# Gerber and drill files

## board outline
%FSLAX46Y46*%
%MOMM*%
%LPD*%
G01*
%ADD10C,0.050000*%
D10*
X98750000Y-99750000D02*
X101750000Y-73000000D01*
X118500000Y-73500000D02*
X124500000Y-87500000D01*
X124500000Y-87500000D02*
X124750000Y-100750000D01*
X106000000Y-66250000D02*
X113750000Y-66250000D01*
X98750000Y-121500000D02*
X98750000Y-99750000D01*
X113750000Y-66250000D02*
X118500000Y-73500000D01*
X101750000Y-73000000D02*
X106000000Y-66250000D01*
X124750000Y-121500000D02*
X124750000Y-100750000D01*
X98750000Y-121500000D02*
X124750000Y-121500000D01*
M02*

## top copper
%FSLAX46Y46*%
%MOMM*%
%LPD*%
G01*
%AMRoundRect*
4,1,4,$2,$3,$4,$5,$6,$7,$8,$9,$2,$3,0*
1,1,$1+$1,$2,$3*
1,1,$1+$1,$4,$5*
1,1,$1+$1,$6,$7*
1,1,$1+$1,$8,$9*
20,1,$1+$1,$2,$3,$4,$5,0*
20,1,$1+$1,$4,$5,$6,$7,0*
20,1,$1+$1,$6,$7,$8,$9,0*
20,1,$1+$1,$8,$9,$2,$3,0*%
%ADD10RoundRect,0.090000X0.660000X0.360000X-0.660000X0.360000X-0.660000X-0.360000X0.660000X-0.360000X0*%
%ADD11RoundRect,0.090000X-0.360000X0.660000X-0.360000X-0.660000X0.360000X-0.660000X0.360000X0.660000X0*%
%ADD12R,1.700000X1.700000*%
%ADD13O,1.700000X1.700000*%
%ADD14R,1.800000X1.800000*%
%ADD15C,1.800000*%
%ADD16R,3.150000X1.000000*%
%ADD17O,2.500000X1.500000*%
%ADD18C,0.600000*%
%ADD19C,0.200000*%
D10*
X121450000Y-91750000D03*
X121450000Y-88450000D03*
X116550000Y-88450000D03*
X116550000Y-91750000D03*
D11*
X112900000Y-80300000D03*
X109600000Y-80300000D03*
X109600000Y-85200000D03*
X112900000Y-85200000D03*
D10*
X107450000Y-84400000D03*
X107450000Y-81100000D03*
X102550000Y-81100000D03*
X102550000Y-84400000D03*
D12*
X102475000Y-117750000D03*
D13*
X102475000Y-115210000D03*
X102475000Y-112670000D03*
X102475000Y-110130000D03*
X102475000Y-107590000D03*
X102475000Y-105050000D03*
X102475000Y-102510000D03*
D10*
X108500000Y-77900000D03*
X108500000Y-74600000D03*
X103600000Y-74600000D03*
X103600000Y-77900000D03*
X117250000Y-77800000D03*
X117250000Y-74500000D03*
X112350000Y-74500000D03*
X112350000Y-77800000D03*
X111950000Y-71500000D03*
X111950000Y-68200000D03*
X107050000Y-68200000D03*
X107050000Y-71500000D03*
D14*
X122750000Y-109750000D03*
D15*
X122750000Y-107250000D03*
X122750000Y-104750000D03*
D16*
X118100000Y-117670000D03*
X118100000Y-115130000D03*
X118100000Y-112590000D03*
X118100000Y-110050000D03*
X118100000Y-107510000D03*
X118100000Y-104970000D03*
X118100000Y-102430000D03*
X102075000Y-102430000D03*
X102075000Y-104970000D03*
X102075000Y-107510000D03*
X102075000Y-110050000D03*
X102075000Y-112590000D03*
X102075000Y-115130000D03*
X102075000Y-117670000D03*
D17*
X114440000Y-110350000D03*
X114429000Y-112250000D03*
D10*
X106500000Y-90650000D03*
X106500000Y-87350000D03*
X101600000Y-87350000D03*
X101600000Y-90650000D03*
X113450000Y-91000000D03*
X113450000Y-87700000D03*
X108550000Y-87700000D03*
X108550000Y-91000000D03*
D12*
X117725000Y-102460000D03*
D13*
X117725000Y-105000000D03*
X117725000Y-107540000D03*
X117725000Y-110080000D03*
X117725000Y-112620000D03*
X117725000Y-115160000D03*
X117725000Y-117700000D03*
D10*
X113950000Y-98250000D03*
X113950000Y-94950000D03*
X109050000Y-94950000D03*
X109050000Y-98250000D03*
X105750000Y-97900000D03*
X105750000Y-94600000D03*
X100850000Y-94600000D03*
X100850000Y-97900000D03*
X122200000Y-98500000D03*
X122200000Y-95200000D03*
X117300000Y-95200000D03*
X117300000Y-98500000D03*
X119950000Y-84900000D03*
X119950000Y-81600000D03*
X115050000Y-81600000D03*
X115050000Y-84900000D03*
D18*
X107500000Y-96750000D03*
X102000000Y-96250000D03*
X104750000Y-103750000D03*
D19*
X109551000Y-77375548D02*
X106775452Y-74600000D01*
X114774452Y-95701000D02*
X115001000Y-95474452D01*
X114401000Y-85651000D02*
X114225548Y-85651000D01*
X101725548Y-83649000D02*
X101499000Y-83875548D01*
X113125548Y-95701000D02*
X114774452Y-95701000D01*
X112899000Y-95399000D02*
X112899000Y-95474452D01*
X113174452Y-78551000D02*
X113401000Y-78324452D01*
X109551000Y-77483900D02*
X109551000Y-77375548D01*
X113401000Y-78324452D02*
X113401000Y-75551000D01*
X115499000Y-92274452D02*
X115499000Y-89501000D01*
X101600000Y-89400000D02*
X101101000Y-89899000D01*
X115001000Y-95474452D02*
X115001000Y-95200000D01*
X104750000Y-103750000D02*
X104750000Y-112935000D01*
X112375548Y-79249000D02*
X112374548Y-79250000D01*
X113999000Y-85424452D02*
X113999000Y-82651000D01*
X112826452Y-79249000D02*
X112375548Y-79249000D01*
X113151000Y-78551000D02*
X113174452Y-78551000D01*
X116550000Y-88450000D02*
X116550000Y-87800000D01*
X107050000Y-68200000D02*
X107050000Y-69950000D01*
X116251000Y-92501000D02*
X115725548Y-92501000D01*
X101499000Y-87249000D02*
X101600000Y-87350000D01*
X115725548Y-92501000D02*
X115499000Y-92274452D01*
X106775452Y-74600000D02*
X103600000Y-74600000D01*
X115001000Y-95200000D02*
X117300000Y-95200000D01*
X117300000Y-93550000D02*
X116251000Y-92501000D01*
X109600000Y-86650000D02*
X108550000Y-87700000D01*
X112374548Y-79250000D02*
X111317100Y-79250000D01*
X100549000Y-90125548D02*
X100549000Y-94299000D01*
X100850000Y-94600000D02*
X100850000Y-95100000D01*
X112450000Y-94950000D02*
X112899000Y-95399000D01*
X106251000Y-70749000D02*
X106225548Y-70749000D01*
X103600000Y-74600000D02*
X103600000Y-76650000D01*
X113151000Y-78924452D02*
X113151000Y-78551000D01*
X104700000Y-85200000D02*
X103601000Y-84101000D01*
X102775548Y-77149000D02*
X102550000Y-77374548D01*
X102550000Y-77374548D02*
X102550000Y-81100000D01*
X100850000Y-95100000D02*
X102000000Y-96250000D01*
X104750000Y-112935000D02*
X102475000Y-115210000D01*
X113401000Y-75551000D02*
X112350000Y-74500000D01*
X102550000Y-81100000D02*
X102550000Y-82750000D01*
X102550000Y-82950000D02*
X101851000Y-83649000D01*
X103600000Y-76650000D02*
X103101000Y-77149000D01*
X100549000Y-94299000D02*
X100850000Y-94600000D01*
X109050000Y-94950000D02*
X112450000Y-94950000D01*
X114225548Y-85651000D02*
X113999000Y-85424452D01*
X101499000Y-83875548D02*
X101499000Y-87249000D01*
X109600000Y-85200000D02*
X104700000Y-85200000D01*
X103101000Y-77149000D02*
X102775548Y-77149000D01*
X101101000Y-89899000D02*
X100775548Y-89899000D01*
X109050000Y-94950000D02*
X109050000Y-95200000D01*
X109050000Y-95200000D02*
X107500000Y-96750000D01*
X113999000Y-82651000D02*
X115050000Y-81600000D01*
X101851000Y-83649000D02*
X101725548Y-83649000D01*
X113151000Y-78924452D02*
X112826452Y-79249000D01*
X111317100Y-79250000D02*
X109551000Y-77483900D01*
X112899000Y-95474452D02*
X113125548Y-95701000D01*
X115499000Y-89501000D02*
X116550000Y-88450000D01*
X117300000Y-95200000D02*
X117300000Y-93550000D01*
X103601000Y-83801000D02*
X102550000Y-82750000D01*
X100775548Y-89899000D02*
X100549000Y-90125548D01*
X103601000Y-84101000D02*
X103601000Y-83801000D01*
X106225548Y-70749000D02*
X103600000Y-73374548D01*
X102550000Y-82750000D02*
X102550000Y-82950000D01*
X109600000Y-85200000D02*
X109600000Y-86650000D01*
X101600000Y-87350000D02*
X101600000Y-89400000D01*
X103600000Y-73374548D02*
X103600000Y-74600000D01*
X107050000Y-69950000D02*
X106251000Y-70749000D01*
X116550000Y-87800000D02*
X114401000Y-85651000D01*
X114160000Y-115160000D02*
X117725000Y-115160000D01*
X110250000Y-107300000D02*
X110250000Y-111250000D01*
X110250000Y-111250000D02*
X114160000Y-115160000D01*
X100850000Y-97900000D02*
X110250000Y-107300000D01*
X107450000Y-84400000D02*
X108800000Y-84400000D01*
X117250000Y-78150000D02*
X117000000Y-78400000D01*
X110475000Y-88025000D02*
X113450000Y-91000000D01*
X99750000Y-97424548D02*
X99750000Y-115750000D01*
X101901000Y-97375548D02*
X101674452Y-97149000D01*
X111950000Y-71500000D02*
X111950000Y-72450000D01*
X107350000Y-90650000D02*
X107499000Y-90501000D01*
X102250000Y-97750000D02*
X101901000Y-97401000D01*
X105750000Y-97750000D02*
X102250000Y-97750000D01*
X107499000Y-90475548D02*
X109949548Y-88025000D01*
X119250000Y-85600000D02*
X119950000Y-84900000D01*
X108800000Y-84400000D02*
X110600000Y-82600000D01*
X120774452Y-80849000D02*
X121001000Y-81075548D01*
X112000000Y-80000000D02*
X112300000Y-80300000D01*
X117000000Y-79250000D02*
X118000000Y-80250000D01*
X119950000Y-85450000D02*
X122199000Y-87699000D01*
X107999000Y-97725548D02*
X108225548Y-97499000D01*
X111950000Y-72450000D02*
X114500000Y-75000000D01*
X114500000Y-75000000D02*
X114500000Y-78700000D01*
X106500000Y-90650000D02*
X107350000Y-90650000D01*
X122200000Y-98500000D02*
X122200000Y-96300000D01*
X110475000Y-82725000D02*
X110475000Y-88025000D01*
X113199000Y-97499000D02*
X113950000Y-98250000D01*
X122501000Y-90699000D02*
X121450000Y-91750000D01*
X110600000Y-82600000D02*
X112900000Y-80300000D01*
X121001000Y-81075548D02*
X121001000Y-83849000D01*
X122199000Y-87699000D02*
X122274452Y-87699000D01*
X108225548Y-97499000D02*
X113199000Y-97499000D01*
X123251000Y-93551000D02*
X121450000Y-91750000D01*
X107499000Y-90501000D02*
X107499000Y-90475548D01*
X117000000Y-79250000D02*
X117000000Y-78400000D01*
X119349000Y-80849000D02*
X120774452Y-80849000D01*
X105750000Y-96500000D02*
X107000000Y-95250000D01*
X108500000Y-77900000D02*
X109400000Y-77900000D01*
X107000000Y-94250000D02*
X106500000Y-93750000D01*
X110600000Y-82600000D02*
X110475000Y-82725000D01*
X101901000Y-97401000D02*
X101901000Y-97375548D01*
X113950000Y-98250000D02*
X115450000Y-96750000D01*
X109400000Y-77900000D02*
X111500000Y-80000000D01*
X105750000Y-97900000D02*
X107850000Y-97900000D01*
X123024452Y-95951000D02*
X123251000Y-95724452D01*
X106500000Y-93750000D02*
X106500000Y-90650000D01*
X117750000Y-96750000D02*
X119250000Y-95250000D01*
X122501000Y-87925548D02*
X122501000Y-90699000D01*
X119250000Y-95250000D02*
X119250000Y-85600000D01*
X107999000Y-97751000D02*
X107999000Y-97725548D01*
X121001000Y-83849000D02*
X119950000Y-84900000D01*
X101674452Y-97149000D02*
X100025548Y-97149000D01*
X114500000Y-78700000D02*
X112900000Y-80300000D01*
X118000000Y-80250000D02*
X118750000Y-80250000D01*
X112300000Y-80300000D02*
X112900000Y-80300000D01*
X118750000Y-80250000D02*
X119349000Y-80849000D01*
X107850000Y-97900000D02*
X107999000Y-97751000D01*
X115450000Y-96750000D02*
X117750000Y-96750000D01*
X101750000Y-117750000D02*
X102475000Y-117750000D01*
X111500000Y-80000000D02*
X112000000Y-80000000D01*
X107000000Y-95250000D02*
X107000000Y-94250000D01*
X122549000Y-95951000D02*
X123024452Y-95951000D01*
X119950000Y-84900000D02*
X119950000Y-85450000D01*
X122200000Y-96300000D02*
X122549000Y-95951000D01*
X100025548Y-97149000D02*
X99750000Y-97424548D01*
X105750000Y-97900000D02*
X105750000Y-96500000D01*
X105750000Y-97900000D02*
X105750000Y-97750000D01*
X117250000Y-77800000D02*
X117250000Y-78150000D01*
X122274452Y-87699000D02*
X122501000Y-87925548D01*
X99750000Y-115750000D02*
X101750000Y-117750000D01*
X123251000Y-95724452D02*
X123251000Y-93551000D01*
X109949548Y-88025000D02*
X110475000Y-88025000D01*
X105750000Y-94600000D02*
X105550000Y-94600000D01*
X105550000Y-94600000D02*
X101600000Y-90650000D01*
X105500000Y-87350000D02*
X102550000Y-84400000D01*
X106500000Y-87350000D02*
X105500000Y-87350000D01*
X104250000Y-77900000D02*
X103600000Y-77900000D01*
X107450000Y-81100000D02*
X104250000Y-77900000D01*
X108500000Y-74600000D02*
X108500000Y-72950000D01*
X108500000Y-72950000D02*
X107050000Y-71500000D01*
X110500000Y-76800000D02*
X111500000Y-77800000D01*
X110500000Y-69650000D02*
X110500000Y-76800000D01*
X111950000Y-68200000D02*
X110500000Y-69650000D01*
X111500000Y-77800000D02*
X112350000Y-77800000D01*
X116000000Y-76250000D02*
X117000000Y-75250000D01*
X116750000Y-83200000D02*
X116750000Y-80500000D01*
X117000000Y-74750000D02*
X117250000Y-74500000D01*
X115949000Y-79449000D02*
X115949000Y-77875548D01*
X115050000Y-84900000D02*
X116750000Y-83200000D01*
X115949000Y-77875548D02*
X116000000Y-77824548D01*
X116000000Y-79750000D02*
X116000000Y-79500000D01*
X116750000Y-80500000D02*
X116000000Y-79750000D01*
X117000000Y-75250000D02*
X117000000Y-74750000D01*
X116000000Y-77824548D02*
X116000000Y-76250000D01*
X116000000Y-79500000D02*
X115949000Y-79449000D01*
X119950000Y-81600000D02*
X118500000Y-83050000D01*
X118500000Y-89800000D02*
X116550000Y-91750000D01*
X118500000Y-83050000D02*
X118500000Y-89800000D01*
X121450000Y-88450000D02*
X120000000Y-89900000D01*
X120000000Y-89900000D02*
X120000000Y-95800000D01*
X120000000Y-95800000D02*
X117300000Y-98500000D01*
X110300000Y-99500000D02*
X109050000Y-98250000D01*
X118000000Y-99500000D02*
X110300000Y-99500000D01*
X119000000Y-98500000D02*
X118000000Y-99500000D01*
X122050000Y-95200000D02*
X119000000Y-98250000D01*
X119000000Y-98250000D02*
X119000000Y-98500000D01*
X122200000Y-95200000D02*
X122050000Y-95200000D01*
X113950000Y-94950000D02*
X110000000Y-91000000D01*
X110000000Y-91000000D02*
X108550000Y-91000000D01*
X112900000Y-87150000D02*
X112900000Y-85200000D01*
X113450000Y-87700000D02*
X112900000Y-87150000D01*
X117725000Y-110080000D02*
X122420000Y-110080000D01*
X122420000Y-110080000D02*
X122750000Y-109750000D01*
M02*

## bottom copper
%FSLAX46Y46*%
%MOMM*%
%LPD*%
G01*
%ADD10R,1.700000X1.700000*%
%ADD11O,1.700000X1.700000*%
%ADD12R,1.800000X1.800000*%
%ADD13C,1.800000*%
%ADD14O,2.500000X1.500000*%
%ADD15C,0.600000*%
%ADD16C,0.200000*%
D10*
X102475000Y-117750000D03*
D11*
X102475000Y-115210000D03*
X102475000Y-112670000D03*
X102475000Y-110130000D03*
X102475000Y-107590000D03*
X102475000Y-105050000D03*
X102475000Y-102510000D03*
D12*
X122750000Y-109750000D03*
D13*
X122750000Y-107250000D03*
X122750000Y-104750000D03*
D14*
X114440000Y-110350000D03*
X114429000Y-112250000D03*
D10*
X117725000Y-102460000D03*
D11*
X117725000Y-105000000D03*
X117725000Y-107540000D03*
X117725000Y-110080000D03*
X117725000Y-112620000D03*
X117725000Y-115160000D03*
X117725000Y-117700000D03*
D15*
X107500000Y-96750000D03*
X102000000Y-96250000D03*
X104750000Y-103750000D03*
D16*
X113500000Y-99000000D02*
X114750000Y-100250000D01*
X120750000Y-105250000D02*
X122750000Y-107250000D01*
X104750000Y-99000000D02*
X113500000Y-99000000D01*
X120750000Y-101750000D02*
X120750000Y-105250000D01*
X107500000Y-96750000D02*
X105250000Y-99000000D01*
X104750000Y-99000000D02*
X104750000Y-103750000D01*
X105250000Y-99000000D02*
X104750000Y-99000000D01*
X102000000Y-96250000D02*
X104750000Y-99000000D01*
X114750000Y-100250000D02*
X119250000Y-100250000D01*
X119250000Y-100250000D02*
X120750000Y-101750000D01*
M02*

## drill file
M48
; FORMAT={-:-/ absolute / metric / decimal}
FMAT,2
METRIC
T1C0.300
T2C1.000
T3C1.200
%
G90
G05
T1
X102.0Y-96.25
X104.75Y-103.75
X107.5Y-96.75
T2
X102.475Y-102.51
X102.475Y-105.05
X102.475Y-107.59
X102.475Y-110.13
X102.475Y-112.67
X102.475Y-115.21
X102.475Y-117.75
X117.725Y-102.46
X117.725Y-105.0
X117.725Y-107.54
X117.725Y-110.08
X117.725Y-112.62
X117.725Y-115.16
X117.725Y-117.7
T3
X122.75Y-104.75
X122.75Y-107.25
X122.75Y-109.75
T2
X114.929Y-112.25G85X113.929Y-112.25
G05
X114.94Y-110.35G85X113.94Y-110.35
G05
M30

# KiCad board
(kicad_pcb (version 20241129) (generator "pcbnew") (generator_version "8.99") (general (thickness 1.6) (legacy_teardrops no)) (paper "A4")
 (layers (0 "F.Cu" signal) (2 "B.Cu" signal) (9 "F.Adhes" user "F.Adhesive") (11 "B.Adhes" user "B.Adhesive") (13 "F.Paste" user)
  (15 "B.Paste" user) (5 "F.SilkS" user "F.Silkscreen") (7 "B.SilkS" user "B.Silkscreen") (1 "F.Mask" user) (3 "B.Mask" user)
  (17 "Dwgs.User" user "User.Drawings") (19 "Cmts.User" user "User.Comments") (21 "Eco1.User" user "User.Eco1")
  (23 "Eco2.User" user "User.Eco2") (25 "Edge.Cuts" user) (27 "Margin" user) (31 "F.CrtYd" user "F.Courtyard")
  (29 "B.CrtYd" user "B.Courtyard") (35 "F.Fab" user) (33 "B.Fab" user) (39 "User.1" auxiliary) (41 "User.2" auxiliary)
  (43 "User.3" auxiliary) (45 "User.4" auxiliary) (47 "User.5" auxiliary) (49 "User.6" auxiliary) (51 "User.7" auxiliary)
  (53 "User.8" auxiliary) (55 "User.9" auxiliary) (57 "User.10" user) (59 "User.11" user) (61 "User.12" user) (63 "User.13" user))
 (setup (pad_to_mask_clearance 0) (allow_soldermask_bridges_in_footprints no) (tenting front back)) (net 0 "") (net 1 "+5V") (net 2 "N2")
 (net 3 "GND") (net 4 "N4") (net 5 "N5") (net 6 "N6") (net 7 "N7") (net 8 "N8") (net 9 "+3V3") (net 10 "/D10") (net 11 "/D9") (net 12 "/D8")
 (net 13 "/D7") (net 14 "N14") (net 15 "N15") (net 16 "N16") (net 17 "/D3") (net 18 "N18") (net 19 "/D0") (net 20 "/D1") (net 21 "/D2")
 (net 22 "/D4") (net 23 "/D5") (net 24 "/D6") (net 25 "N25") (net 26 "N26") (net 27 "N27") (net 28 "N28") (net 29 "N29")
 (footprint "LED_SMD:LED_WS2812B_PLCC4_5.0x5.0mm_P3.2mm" (layer "F.Cu") (at 119 90.1 180)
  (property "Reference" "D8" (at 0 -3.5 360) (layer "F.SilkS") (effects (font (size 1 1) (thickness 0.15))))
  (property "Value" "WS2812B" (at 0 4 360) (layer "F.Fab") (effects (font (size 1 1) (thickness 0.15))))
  (pad "1" smd roundrect (at -2.45 -1.65 180) (size 1.5 0.9) (layers "F.Cu" "F.Mask" "F.Paste") (roundrect_rratio 0.1) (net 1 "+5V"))
  (pad "2" smd roundrect (at -2.45 1.65 180) (size 1.5 0.9) (layers "F.Cu" "F.Mask" "F.Paste") (roundrect_rratio 0.1) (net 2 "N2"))
  (pad "3" smd roundrect (at 2.45 1.65 180) (size 1.5 0.9) (layers "F.Cu" "F.Mask" "F.Paste") (roundrect_rratio 0.1) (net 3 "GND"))
  (pad "4" smd roundrect (at 2.45 -1.65 180) (size 1.5 0.9) (layers "F.Cu" "F.Mask" "F.Paste") (roundrect_rratio 0.1) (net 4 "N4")))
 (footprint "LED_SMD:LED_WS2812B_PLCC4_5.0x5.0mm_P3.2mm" (layer "F.Cu") (at 111.25 82.75 -90)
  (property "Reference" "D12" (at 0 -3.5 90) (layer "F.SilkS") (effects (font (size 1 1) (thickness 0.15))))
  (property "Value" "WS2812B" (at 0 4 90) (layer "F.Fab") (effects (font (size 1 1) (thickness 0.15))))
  (pad "1" smd roundrect (at -2.45 -1.65 270) (size 1.5 0.9) (layers "F.Cu" "F.Mask" "F.Paste") (roundrect_rratio 0.1) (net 1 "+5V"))
  (pad "2" smd roundrect (at -2.45 1.65 270) (size 1.5 0.9) (layers "F.Cu" "F.Mask" "F.Paste") (roundrect_rratio 0.1) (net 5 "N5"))
  (pad "3" smd roundrect (at 2.45 1.65 270) (size 1.5 0.9) (layers "F.Cu" "F.Mask" "F.Paste") (roundrect_rratio 0.1) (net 3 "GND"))
  (pad "4" smd roundrect (at 2.45 -1.65 270) (size 1.5 0.9) (layers "F.Cu" "F.Mask" "F.Paste") (roundrect_rratio 0.1) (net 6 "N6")))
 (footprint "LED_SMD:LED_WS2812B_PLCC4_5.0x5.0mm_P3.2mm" (layer "F.Cu") (at 105 82.75 180)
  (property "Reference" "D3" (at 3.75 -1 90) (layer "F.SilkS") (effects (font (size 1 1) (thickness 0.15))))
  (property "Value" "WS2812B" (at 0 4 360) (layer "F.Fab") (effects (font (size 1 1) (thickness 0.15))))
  (pad "1" smd roundrect (at -2.45 -1.65 180) (size 1.5 0.9) (layers "F.Cu" "F.Mask" "F.Paste") (roundrect_rratio 0.1) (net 1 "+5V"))
  (pad "2" smd roundrect (at -2.45 1.65 180) (size 1.5 0.9) (layers "F.Cu" "F.Mask" "F.Paste") (roundrect_rratio 0.1) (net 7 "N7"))
  (pad "3" smd roundrect (at 2.45 1.65 180) (size 1.5 0.9) (layers "F.Cu" "F.Mask" "F.Paste") (roundrect_rratio 0.1) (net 3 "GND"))
  (pad "4" smd roundrect (at 2.45 -1.65 180) (size 1.5 0.9) (layers "F.Cu" "F.Mask" "F.Paste") (roundrect_rratio 0.1) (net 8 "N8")))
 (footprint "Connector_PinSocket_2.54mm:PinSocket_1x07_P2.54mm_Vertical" (layer "F.Cu") (at 102.475 117.75 180)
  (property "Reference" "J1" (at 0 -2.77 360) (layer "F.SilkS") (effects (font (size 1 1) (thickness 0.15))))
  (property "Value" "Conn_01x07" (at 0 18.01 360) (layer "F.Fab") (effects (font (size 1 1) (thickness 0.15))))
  (pad "1" thru_hole rect (at 0 0 180) (size 1.7 1.7) (drill 1) (layers "*.Cu" "*.Mask") (remove_unused_layers no) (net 1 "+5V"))
  (pad "2" thru_hole oval (at 0 2.54 180) (size 1.7 1.7) (drill 1) (layers "*.Cu" "*.Mask") (remove_unused_layers no) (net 3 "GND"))
  (pad "3" thru_hole oval (at 0 5.08 180) (size 1.7 1.7) (drill 1) (layers "*.Cu" "*.Mask") (remove_unused_layers no) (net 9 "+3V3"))
  (pad "4" thru_hole oval (at 0 7.62 180) (size 1.7 1.7) (drill 1) (layers "*.Cu" "*.Mask") (remove_unused_layers no) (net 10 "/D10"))
  (pad "5" thru_hole oval (at 0 10.16 180) (size 1.7 1.7) (drill 1) (layers "*.Cu" "*.Mask") (remove_unused_layers no) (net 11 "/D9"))
  (pad "6" thru_hole oval (at 0 12.7 180) (size 1.7 1.7) (drill 1) (layers "*.Cu" "*.Mask") (remove_unused_layers no) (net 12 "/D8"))
  (pad "7" thru_hole oval (at 0 15.24 180) (size 1.7 1.7) (drill 1) (layers "*.Cu" "*.Mask") (remove_unused_layers no) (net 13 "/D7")))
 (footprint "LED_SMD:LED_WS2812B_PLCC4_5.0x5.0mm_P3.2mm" (layer "F.Cu") (at 106.05 76.25 180)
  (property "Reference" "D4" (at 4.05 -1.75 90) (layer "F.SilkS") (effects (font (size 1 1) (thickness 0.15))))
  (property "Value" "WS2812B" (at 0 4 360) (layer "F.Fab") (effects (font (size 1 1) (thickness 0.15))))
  (pad "1" smd roundrect (at -2.45 -1.65 180) (size 1.5 0.9) (layers "F.Cu" "F.Mask" "F.Paste") (roundrect_rratio 0.1) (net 1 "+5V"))
  (pad "2" smd roundrect (at -2.45 1.65 180) (size 1.5 0.9) (layers "F.Cu" "F.Mask" "F.Paste") (roundrect_rratio 0.1) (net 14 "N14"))
  (pad "3" smd roundrect (at 2.45 1.65 180) (size 1.5 0.9) (layers "F.Cu" "F.Mask" "F.Paste") (roundrect_rratio 0.1) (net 3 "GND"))
  (pad "4" smd roundrect (at 2.45 -1.65 180) (size 1.5 0.9) (layers "F.Cu" "F.Mask" "F.Paste") (roundrect_rratio 0.1) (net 7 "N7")))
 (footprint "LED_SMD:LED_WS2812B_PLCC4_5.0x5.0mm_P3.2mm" (layer "F.Cu") (at 114.8 76.15 180)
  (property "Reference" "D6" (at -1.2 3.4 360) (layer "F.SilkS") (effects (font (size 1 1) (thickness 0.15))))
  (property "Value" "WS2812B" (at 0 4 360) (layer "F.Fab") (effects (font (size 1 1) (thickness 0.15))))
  (pad "1" smd roundrect (at -2.45 -1.65 180) (size 1.5 0.9) (layers "F.Cu" "F.Mask" "F.Paste") (roundrect_rratio 0.1) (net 1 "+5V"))
  (pad "2" smd roundrect (at -2.45 1.65 180) (size 1.5 0.9) (layers "F.Cu" "F.Mask" "F.Paste") (roundrect_rratio 0.1) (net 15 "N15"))
  (pad "3" smd roundrect (at 2.45 1.65 180) (size 1.5 0.9) (layers "F.Cu" "F.Mask" "F.Paste") (roundrect_rratio 0.1) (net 3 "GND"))
  (pad "4" smd roundrect (at 2.45 -1.65 180) (size 1.5 0.9) (layers "F.Cu" "F.Mask" "F.Paste") (roundrect_rratio 0.1) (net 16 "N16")))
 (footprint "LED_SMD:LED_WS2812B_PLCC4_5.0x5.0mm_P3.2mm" (layer "F.Cu") (at 109.5 69.85 180)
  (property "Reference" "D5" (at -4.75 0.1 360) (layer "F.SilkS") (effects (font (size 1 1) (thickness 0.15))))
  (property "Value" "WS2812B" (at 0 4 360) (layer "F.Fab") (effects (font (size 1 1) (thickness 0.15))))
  (pad "1" smd roundrect (at -2.45 -1.65 180) (size 1.5 0.9) (layers "F.Cu" "F.Mask" "F.Paste") (roundrect_rratio 0.1) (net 1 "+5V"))
  (pad "2" smd roundrect (at -2.45 1.65 180) (size 1.5 0.9) (layers "F.Cu" "F.Mask" "F.Paste") (roundrect_rratio 0.1) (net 16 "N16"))
  (pad "3" smd roundrect (at 2.45 1.65 180) (size 1.5 0.9) (layers "F.Cu" "F.Mask" "F.Paste") (roundrect_rratio 0.1) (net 3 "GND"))
  (pad "4" smd roundrect (at 2.45 -1.65 180) (size 1.5 0.9) (layers "F.Cu" "F.Mask" "F.Paste") (roundrect_rratio 0.1) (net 14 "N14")))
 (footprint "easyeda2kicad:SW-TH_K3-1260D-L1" (layer "F.Cu") (at 122.75 107.25 180)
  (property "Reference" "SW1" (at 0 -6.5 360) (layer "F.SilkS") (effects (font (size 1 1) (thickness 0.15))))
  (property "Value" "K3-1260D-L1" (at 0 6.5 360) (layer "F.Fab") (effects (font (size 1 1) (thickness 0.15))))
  (pad "1" thru_hole rect (at 0 -2.5 90) (size 1.8 1.8) (drill 1.199998) (layers "*.Cu" "*.Mask") (remove_unused_layers no) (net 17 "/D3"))
  (pad "2" thru_hole circle (at 0 0 90) (size 1.8 1.8) (drill 1.199998) (layers "*.Cu" "*.Mask") (remove_unused_layers no) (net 3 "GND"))
  (pad "3" thru_hole circle (at 0 2.5 90) (size 1.8 1.8) (drill 1.199998) (layers "*.Cu" "*.Mask") (remove_unused_layers no) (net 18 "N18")))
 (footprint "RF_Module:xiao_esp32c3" (layer "F.Cu") (at 109.5 108.25 180)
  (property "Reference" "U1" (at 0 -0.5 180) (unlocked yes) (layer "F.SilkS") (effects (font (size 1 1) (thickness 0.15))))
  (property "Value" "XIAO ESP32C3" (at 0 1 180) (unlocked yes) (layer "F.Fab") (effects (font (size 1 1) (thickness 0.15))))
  (pad "1" smd rect (at -8.6 -9.42 180) (size 3.15 1) (layers "F.Cu" "F.Mask" "F.Paste") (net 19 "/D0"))
  (pad "2" smd rect (at -8.6 -6.88 180) (size 3.15 1) (layers "F.Cu" "F.Mask" "F.Paste") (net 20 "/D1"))
  (pad "3" smd rect (at -8.6 -4.34 180) (size 3.15 1) (layers "F.Cu" "F.Mask" "F.Paste") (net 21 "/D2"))
  (pad "4" smd rect (at -8.6 -1.8 180) (size 3.15 1) (layers "F.Cu" "F.Mask" "F.Paste") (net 17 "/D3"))
  (pad "5" smd rect (at -8.6 0.74 180) (size 3.15 1) (layers "F.Cu" "F.Mask" "F.Paste") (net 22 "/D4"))
  (pad "6" smd rect (at -8.6 3.28 180) (size 3.15 1) (layers "F.Cu" "F.Mask" "F.Paste") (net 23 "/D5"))
  (pad "7" smd rect (at -8.6 5.82 180) (size 3.15 1) (layers "F.Cu" "F.Mask" "F.Paste") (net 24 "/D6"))
  (pad "8" smd rect (at 7.425 5.82 180) (size 3.15 1) (layers "F.Cu" "F.Mask" "F.Paste") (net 13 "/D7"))
  (pad "9" smd rect (at 7.425 3.28 180) (size 3.15 1) (layers "F.Cu" "F.Mask" "F.Paste") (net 12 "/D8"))
  (pad "10" smd rect (at 7.425 0.74 180) (size 3.15 1) (layers "F.Cu" "F.Mask" "F.Paste") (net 11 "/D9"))
  (pad "11" smd rect (at 7.425 -1.8 180) (size 3.15 1) (layers "F.Cu" "F.Mask" "F.Paste") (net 10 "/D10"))
  (pad "12" smd rect (at 7.425 -4.34 180) (size 3.15 1) (layers "F.Cu" "F.Mask" "F.Paste") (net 9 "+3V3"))
  (pad "13" smd rect (at 7.425 -6.88 180) (size 3.15 1) (layers "F.Cu" "F.Mask" "F.Paste") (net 3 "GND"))
  (pad "14" smd rect (at 7.425 -9.42 180) (size 3.15 1) (layers "F.Cu" "F.Mask" "F.Paste") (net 1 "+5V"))
  (pad "B+" thru_hole oval (at -4.94 -2.1 180) (size 2.5 1.5) (drill oval 2 1) (layers "*.Cu" "*.Mask") (remove_unused_layers no)
   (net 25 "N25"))
  (pad "B-" thru_hole oval (at -4.929 -4 180) (size 2.5 1.5) (drill oval 2 1) (layers "*.Cu" "*.Mask") (remove_unused_layers no)
   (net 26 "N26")))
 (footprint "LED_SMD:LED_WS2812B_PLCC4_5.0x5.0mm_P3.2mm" (layer "F.Cu") (at 104.05 89 180)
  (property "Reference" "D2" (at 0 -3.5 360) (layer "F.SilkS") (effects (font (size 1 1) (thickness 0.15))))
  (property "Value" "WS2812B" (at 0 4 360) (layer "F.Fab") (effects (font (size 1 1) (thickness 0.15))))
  (pad "1" smd roundrect (at -2.45 -1.65 180) (size 1.5 0.9) (layers "F.Cu" "F.Mask" "F.Paste") (roundrect_rratio 0.1) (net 1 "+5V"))
  (pad "2" smd roundrect (at -2.45 1.65 180) (size 1.5 0.9) (layers "F.Cu" "F.Mask" "F.Paste") (roundrect_rratio 0.1) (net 8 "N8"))
  (pad "3" smd roundrect (at 2.45 1.65 180) (size 1.5 0.9) (layers "F.Cu" "F.Mask" "F.Paste") (roundrect_rratio 0.1) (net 3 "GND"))
  (pad "4" smd roundrect (at 2.45 -1.65 180) (size 1.5 0.9) (layers "F.Cu" "F.Mask" "F.Paste") (roundrect_rratio 0.1) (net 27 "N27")))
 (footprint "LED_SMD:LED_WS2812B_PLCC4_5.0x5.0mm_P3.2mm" (layer "F.Cu") (at 111 89.35 180)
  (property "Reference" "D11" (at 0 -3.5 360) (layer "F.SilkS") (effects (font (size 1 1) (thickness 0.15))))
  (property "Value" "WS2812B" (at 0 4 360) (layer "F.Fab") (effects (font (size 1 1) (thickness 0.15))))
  (pad "1" smd roundrect (at -2.45 -1.65 180) (size 1.5 0.9) (layers "F.Cu" "F.Mask" "F.Paste") (roundrect_rratio 0.1) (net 1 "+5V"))
  (pad "2" smd roundrect (at -2.45 1.65 180) (size 1.5 0.9) (layers "F.Cu" "F.Mask" "F.Paste") (roundrect_rratio 0.1) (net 6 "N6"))
  (pad "3" smd roundrect (at 2.45 1.65 180) (size 1.5 0.9) (layers "F.Cu" "F.Mask" "F.Paste") (roundrect_rratio 0.1) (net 3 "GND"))
  (pad "4" smd roundrect (at 2.45 -1.65 180) (size 1.5 0.9) (layers "F.Cu" "F.Mask" "F.Paste") (roundrect_rratio 0.1) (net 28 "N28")))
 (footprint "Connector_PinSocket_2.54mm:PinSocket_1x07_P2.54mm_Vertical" (layer "F.Cu") (at 117.725 102.46)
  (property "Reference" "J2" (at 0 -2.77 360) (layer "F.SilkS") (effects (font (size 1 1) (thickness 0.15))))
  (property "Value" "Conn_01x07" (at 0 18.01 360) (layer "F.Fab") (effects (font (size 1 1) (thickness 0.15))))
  (pad "1" thru_hole rect (at 0 0) (size 1.7 1.7) (drill 1) (layers "*.Cu" "*.Mask") (remove_unused_layers no) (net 24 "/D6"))
  (pad "2" thru_hole oval (at 0 2.54) (size 1.7 1.7) (drill 1) (layers "*.Cu" "*.Mask") (remove_unused_layers no) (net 23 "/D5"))
  (pad "3" thru_hole oval (at 0 5.08) (size 1.7 1.7) (drill 1) (layers "*.Cu" "*.Mask") (remove_unused_layers no) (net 22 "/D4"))
  (pad "4" thru_hole oval (at 0 7.62) (size 1.7 1.7) (drill 1) (layers "*.Cu" "*.Mask") (remove_unused_layers no) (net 17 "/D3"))
  (pad "5" thru_hole oval (at 0 10.16) (size 1.7 1.7) (drill 1) (layers "*.Cu" "*.Mask") (remove_unused_layers no) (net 21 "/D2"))
  (pad "6" thru_hole oval (at 0 12.7) (size 1.7 1.7) (drill 1) (layers "*.Cu" "*.Mask") (remove_unused_layers no) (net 20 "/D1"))
  (pad "7" thru_hole oval (at 0 15.24) (size 1.7 1.7) (drill 1) (layers "*.Cu" "*.Mask") (remove_unused_layers no) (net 19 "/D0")))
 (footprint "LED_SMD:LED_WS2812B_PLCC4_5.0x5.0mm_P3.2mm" (layer "F.Cu") (at 111.5 96.6 180)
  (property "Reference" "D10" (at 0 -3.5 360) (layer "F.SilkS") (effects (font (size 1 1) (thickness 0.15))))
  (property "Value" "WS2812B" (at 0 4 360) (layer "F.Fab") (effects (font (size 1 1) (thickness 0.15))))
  (pad "1" smd roundrect (at -2.45 -1.65 180) (size 1.5 0.9) (layers "F.Cu" "F.Mask" "F.Paste") (roundrect_rratio 0.1) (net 1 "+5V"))
  (pad "2" smd roundrect (at -2.45 1.65 180) (size 1.5 0.9) (layers "F.Cu" "F.Mask" "F.Paste") (roundrect_rratio 0.1) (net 28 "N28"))
  (pad "3" smd roundrect (at 2.45 1.65 180) (size 1.5 0.9) (layers "F.Cu" "F.Mask" "F.Paste") (roundrect_rratio 0.1) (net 3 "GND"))
  (pad "4" smd roundrect (at 2.45 -1.65 180) (size 1.5 0.9) (layers "F.Cu" "F.Mask" "F.Paste") (roundrect_rratio 0.1) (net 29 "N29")))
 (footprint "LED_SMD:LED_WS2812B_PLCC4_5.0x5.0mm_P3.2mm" (layer "F.Cu") (at 103.3 96.25 180)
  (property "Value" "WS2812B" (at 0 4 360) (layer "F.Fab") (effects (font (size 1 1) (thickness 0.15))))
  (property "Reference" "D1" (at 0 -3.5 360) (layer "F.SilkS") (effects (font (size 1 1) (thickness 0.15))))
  (pad "1" smd roundrect (at -2.45 -1.65 180) (size 1.5 0.9) (layers "F.Cu" "F.Mask" "F.Paste") (roundrect_rratio 0.1) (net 1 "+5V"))
  (pad "2" smd roundrect (at -2.45 1.65 180) (size 1.5 0.9) (layers "F.Cu" "F.Mask" "F.Paste") (roundrect_rratio 0.1) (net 27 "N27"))
  (pad "3" smd roundrect (at 2.45 1.65 180) (size 1.5 0.9) (layers "F.Cu" "F.Mask" "F.Paste") (roundrect_rratio 0.1) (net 3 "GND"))
  (pad "4" smd roundrect (at 2.45 -1.65 180) (size 1.5 0.9) (layers "F.Cu" "F.Mask" "F.Paste") (roundrect_rratio 0.1) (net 20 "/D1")))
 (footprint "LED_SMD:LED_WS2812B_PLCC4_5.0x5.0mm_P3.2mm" (layer "F.Cu") (at 119.75 96.85 180)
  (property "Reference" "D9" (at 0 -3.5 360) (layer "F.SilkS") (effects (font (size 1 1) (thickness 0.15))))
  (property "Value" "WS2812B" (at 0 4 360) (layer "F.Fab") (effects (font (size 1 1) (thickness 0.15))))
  (pad "1" smd roundrect (at -2.45 -1.65 180) (size 1.5 0.9) (layers "F.Cu" "F.Mask" "F.Paste") (roundrect_rratio 0.1) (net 1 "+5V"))
  (pad "2" smd roundrect (at -2.45 1.65 180) (size 1.5 0.9) (layers "F.Cu" "F.Mask" "F.Paste") (roundrect_rratio 0.1) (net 29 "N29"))
  (pad "3" smd roundrect (at 2.45 1.65 180) (size 1.5 0.9) (layers "F.Cu" "F.Mask" "F.Paste") (roundrect_rratio 0.1) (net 3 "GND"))
  (pad "4" smd roundrect (at 2.45 -1.65 180) (size 1.5 0.9) (layers "F.Cu" "F.Mask" "F.Paste") (roundrect_rratio 0.1) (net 2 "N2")))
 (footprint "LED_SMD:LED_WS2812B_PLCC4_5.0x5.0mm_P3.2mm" (layer "F.Cu") (at 117.5 83.25 180)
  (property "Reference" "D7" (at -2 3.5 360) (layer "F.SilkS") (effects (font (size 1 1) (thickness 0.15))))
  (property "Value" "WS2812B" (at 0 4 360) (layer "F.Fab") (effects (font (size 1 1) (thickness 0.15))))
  (pad "1" smd roundrect (at -2.45 -1.65 180) (size 1.5 0.9) (layers "F.Cu" "F.Mask" "F.Paste") (roundrect_rratio 0.1) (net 1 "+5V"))
  (pad "2" smd roundrect (at -2.45 1.65 180) (size 1.5 0.9) (layers "F.Cu" "F.Mask" "F.Paste") (roundrect_rratio 0.1) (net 4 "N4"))
  (pad "3" smd roundrect (at 2.45 1.65 180) (size 1.5 0.9) (layers "F.Cu" "F.Mask" "F.Paste") (roundrect_rratio 0.1) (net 3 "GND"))
  (pad "4" smd roundrect (at 2.45 -1.65 180) (size 1.5 0.9) (layers "F.Cu" "F.Mask" "F.Paste") (roundrect_rratio 0.1) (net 15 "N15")))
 (gr_line (start 98.75 99.75) (end 101.75 73) (stroke (width 0.05) (type default)) (layer "Edge.Cuts"))
 (gr_line (start 118.5 73.5) (end 124.5 87.5) (stroke (width 0.05) (type default)) (layer "Edge.Cuts"))
 (gr_line (start 124.5 87.5) (end 124.75 100.75) (stroke (width 0.05) (type default)) (layer "Edge.Cuts"))
 (gr_line (start 106 66.25) (end 113.75 66.25) (stroke (width 0.05) (type default)) (layer "Edge.Cuts"))
 (gr_line (start 98.75 121.5) (end 98.75 99.75) (stroke (width 0.05) (type default)) (layer "Edge.Cuts"))
 (gr_line (start 113.75 66.25) (end 118.5 73.5) (stroke (width 0.05) (type default)) (layer "Edge.Cuts"))
 (gr_line (start 101.75 73) (end 106 66.25) (stroke (width 0.05) (type default)) (layer "Edge.Cuts"))
 (gr_line (start 124.75 121.5) (end 124.75 100.75) (stroke (width 0.05) (type default)) (layer "Edge.Cuts"))
 (gr_line (start 98.75 121.5) (end 124.75 121.5) (stroke (width 0.05) (type default)) (layer "Edge.Cuts"))
 (segment (start 109.551 77.375548) (end 106.775452 74.6) (width 0.2) (layer "F.Cu") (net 3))
 (segment (start 114.774452 95.701) (end 115.001 95.474452) (width 0.2) (layer "F.Cu") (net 3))
 (segment (start 114.401 85.651) (end 114.225548 85.651) (width 0.2) (layer "F.Cu") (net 3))
 (segment (start 101.725548 83.649) (end 101.499 83.875548) (width 0.2) (layer "F.Cu") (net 3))
 (segment (start 113.125548 95.701) (end 114.774452 95.701) (width 0.2) (layer "F.Cu") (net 3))
 (segment (start 112.899 95.399) (end 112.899 95.474452) (width 0.2) (layer "F.Cu") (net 3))
 (segment (start 113.174452 78.551) (end 113.401 78.324452) (width 0.2) (layer "F.Cu") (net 3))
 (segment (start 109.551 77.4839) (end 109.551 77.375548) (width 0.2) (layer "F.Cu") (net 3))
 (segment (start 113.401 78.324452) (end 113.401 75.551) (width 0.2) (layer "F.Cu") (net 3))
 (segment (start 115.499 92.274452) (end 115.499 89.501) (width 0.2) (layer "F.Cu") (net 3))
 (segment (start 101.6 89.4) (end 101.101 89.899) (width 0.2) (layer "F.Cu") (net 3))
 (segment (start 115.001 95.474452) (end 115.001 95.2) (width 0.2) (layer "F.Cu") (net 3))
 (segment (start 104.75 103.75) (end 104.75 112.935) (width 0.2) (layer "F.Cu") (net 3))
 (segment (start 112.375548 79.249) (end 112.374548 79.25) (width 0.2) (layer "F.Cu") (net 3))
 (segment (start 113.999 85.424452) (end 113.999 82.651) (width 0.2) (layer "F.Cu") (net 3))
 (segment (start 112.826452 79.249) (end 112.375548 79.249) (width 0.2) (layer "F.Cu") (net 3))
 (segment (start 113.151 78.551) (end 113.174452 78.551) (width 0.2) (layer "F.Cu") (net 3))
 (segment (start 116.55 88.45) (end 116.55 87.8) (width 0.2) (layer "F.Cu") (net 3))
 (segment (start 107.05 68.2) (end 107.05 69.95) (width 0.2) (layer "F.Cu") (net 3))
 (segment (start 116.251 92.501) (end 115.725548 92.501) (width 0.2) (layer "F.Cu") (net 3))
 (segment (start 101.499 87.249) (end 101.6 87.35) (width 0.2) (layer "F.Cu") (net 3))
 (segment (start 115.725548 92.501) (end 115.499 92.274452) (width 0.2) (layer "F.Cu") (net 3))
 (segment (start 106.775452 74.6) (end 103.6 74.6) (width 0.2) (layer "F.Cu") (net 3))
 (segment (start 115.001 95.2) (end 117.3 95.2) (width 0.2) (layer "F.Cu") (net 3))
 (segment (start 117.3 93.55) (end 116.251 92.501) (width 0.2) (layer "F.Cu") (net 3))
 (segment (start 109.6 86.65) (end 108.55 87.7) (width 0.2) (layer "F.Cu") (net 3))
 (segment (start 112.374548 79.25) (end 111.3171 79.25) (width 0.2) (layer "F.Cu") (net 3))
 (segment (start 100.549 90.125548) (end 100.549 94.299) (width 0.2) (layer "F.Cu") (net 3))
 (segment (start 100.85 94.6) (end 100.85 95.1) (width 0.2) (layer "F.Cu") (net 3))
 (segment (start 112.45 94.95) (end 112.899 95.399) (width 0.2) (layer "F.Cu") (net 3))
 (segment (start 106.251 70.749) (end 106.225548 70.749) (width 0.2) (layer "F.Cu") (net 3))
 (segment (start 103.6 74.6) (end 103.6 76.65) (width 0.2) (layer "F.Cu") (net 3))
 (segment (start 113.151 78.924452) (end 113.151 78.551) (width 0.2) (layer "F.Cu") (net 3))
 (segment (start 104.7 85.2) (end 103.601 84.101) (width 0.2) (layer "F.Cu") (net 3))
 (segment (start 102.775548 77.149) (end 102.55 77.374548) (width 0.2) (layer "F.Cu") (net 3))
 (segment (start 102.55 77.374548) (end 102.55 81.1) (width 0.2) (layer "F.Cu") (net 3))
 (segment (start 100.85 95.1) (end 102 96.25) (width 0.2) (layer "F.Cu") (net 3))
 (segment (start 104.75 112.935) (end 102.475 115.21) (width 0.2) (layer "F.Cu") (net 3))
 (segment (start 113.401 75.551) (end 112.35 74.5) (width 0.2) (layer "F.Cu") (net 3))
 (segment (start 102.55 81.1) (end 102.55 82.75) (width 0.2) (layer "F.Cu") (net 3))
 (segment (start 102.55 82.95) (end 101.851 83.649) (width 0.2) (layer "F.Cu") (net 3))
 (segment (start 103.6 76.65) (end 103.101 77.149) (width 0.2) (layer "F.Cu") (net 3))
 (segment (start 100.549 94.299) (end 100.85 94.6) (width 0.2) (layer "F.Cu") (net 3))
 (segment (start 109.05 94.95) (end 112.45 94.95) (width 0.2) (layer "F.Cu") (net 3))
 (segment (start 114.225548 85.651) (end 113.999 85.424452) (width 0.2) (layer "F.Cu") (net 3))
 (segment (start 101.499 83.875548) (end 101.499 87.249) (width 0.2) (layer "F.Cu") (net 3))
 (segment (start 109.6 85.2) (end 104.7 85.2) (width 0.2) (layer "F.Cu") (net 3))
 (segment (start 103.101 77.149) (end 102.775548 77.149) (width 0.2) (layer "F.Cu") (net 3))
 (segment (start 101.101 89.899) (end 100.775548 89.899) (width 0.2) (layer "F.Cu") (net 3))
 (segment (start 109.05 94.95) (end 109.05 95.2) (width 0.2) (layer "F.Cu") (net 3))
 (segment (start 109.05 95.2) (end 107.5 96.75) (width 0.2) (layer "F.Cu") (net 3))
 (segment (start 113.999 82.651) (end 115.05 81.6) (width 0.2) (layer "F.Cu") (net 3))
 (segment (start 101.851 83.649) (end 101.725548 83.649) (width 0.2) (layer "F.Cu") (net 3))
 (segment (start 113.151 78.924452) (end 112.826452 79.249) (width 0.2) (layer "F.Cu") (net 3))
 (segment (start 111.3171 79.25) (end 109.551 77.4839) (width 0.2) (layer "F.Cu") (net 3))
 (segment (start 112.899 95.474452) (end 113.125548 95.701) (width 0.2) (layer "F.Cu") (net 3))
 (segment (start 115.499 89.501) (end 116.55 88.45) (width 0.2) (layer "F.Cu") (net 3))
 (segment (start 117.3 95.2) (end 117.3 93.55) (width 0.2) (layer "F.Cu") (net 3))
 (segment (start 103.601 83.801) (end 102.55 82.75) (width 0.2) (layer "F.Cu") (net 3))
 (segment (start 100.775548 89.899) (end 100.549 90.125548) (width 0.2) (layer "F.Cu") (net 3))
 (segment (start 103.601 84.101) (end 103.601 83.801) (width 0.2) (layer "F.Cu") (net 3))
 (segment (start 106.225548 70.749) (end 103.6 73.374548) (width 0.2) (layer "F.Cu") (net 3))
 (segment (start 102.55 82.75) (end 102.55 82.95) (width 0.2) (layer "F.Cu") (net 3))
 (segment (start 109.6 85.2) (end 109.6 86.65) (width 0.2) (layer "F.Cu") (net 3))
 (segment (start 101.6 87.35) (end 101.6 89.4) (width 0.2) (layer "F.Cu") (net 3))
 (segment (start 103.6 73.374548) (end 103.6 74.6) (width 0.2) (layer "F.Cu") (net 3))
 (segment (start 107.05 69.95) (end 106.251 70.749) (width 0.2) (layer "F.Cu") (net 3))
 (segment (start 116.55 87.8) (end 114.401 85.651) (width 0.2) (layer "F.Cu") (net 3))
 (via (at 107.5 96.75) (size 0.6) (drill 0.3) (layers "F.Cu" "B.Cu") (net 3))
 (via (at 102 96.25) (size 0.6) (drill 0.3) (layers "F.Cu" "B.Cu") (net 3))
 (via (at 104.75 103.75) (size 0.6) (drill 0.3) (layers "F.Cu" "B.Cu") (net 3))
 (segment (start 113.5 99) (end 114.75 100.25) (width 0.2) (layer "B.Cu") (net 3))
 (segment (start 120.75 105.25) (end 122.75 107.25) (width 0.2) (layer "B.Cu") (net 3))
 (segment (start 104.75 99) (end 113.5 99) (width 0.2) (layer "B.Cu") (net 3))
 (segment (start 120.75 101.75) (end 120.75 105.25) (width 0.2) (layer "B.Cu") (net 3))
 (segment (start 107.5 96.75) (end 105.25 99) (width 0.2) (layer "B.Cu") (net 3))
 (segment (start 104.75 99) (end 104.75 103.75) (width 0.2) (layer "B.Cu") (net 3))
 (segment (start 105.25 99) (end 104.75 99) (width 0.2) (layer "B.Cu") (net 3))
 (segment (start 102 96.25) (end 104.75 99) (width 0.2) (layer "B.Cu") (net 3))
 (segment (start 114.75 100.25) (end 119.25 100.25) (width 0.2) (layer "B.Cu") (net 3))
 (segment (start 119.25 100.25) (end 120.75 101.75) (width 0.2) (layer "B.Cu") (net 3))
 (segment (start 114.16 115.16) (end 117.725 115.16) (width 0.2) (layer "F.Cu") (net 20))
 (segment (start 110.25 107.3) (end 110.25 111.25) (width 0.2) (layer "F.Cu") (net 20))
 (segment (start 110.25 111.25) (end 114.16 115.16) (width 0.2) (layer "F.Cu") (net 20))
 (segment (start 100.85 97.9) (end 110.25 107.3) (width 0.2) (layer "F.Cu") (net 20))
 (segment (start 107.45 84.4) (end 108.8 84.4) (width 0.2) (layer "F.Cu") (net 1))
 (segment (start 117.25 78.15) (end 117 78.4) (width 0.2) (layer "F.Cu") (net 1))
 (segment (start 110.475 88.025) (end 113.45 91) (width 0.2) (layer "F.Cu") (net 1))
 (segment (start 99.75 97.424548) (end 99.75 115.75) (width 0.2) (layer "F.Cu") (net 1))
 (segment (start 101.901 97.375548) (end 101.674452 97.149) (width 0.2) (layer "F.Cu") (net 1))
 (segment (start 111.95 71.5) (end 111.95 72.45) (width 0.2) (layer "F.Cu") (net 1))
 (segment (start 107.35 90.65) (end 107.499 90.501) (width 0.2) (layer "F.Cu") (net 1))
 (segment (start 102.25 97.75) (end 101.901 97.401) (width 0.2) (layer "F.Cu") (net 1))
 (segment (start 105.75 97.75) (end 102.25 97.75) (width 0.2) (layer "F.Cu") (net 1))
 (segment (start 107.499 90.475548) (end 109.949548 88.025) (width 0.2) (layer "F.Cu") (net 1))
 (segment (start 119.25 85.6) (end 119.95 84.9) (width 0.2) (layer "F.Cu") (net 1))
 (segment (start 108.8 84.4) (end 110.6 82.6) (width 0.2) (layer "F.Cu") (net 1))
 (segment (start 120.774452 80.849) (end 121.001 81.075548) (width 0.2) (layer "F.Cu") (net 1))
 (segment (start 112 80) (end 112.3 80.3) (width 0.2) (layer "F.Cu") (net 1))
 (segment (start 117 79.25) (end 118 80.25) (width 0.2) (layer "F.Cu") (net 1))
 (segment (start 119.95 85.45) (end 122.199 87.699) (width 0.2) (layer "F.Cu") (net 1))
 (segment (start 107.999 97.725548) (end 108.225548 97.499) (width 0.2) (layer "F.Cu") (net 1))
 (segment (start 111.95 72.45) (end 114.5 75) (width 0.2) (layer "F.Cu") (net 1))
 (segment (start 114.5 75) (end 114.5 78.7) (width 0.2) (layer "F.Cu") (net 1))
 (segment (start 106.5 90.65) (end 107.35 90.65) (width 0.2) (layer "F.Cu") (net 1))
 (segment (start 122.2 98.5) (end 122.2 96.3) (width 0.2) (layer "F.Cu") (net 1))
 (segment (start 110.475 82.725) (end 110.475 88.025) (width 0.2) (layer "F.Cu") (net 1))
 (segment (start 113.199 97.499) (end 113.95 98.25) (width 0.2) (layer "F.Cu") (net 1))
 (segment (start 122.501 90.699) (end 121.45 91.75) (width 0.2) (layer "F.Cu") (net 1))
 (segment (start 110.6 82.6) (end 112.9 80.3) (width 0.2) (layer "F.Cu") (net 1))
 (segment (start 121.001 81.075548) (end 121.001 83.849) (width 0.2) (layer "F.Cu") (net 1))
 (segment (start 122.199 87.699) (end 122.274452 87.699) (width 0.2) (layer "F.Cu") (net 1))
 (segment (start 108.225548 97.499) (end 113.199 97.499) (width 0.2) (layer "F.Cu") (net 1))
 (segment (start 123.251 93.551) (end 121.45 91.75) (width 0.2) (layer "F.Cu") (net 1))
 (segment (start 107.499 90.501) (end 107.499 90.475548) (width 0.2) (layer "F.Cu") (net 1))
 (segment (start 117 79.25) (end 117 78.4) (width 0.2) (layer "F.Cu") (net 1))
 (segment (start 119.349 80.849) (end 120.774452 80.849) (width 0.2) (layer "F.Cu") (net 1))
 (segment (start 105.75 96.5) (end 107 95.25) (width 0.2) (layer "F.Cu") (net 1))
 (segment (start 108.5 77.9) (end 109.4 77.9) (width 0.2) (layer "F.Cu") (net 1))
 (segment (start 107 94.25) (end 106.5 93.75) (width 0.2) (layer "F.Cu") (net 1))
 (segment (start 110.6 82.6) (end 110.475 82.725) (width 0.2) (layer "F.Cu") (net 1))
 (segment (start 101.901 97.401) (end 101.901 97.375548) (width 0.2) (layer "F.Cu") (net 1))
 (segment (start 113.95 98.25) (end 115.45 96.75) (width 0.2) (layer "F.Cu") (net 1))
 (segment (start 109.4 77.9) (end 111.5 80) (width 0.2) (layer "F.Cu") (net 1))
 (segment (start 105.75 97.9) (end 107.85 97.9) (width 0.2) (layer "F.Cu") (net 1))
 (segment (start 123.024452 95.951) (end 123.251 95.724452) (width 0.2) (layer "F.Cu") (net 1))
 (segment (start 106.5 93.75) (end 106.5 90.65) (width 0.2) (layer "F.Cu") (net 1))
 (segment (start 117.75 96.75) (end 119.25 95.25) (width 0.2) (layer "F.Cu") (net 1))
 (segment (start 122.501 87.925548) (end 122.501 90.699) (width 0.2) (layer "F.Cu") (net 1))
 (segment (start 119.25 95.25) (end 119.25 85.6) (width 0.2) (layer "F.Cu") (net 1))
 (segment (start 107.999 97.751) (end 107.999 97.725548) (width 0.2) (layer "F.Cu") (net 1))
 (segment (start 121.001 83.849) (end 119.95 84.9) (width 0.2) (layer "F.Cu") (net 1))
 (segment (start 101.674452 97.149) (end 100.025548 97.149) (width 0.2) (layer "F.Cu") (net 1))
 (segment (start 114.5 78.7) (end 112.9 80.3) (width 0.2) (layer "F.Cu") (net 1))
 (segment (start 118 80.25) (end 118.75 80.25) (width 0.2) (layer "F.Cu") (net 1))
 (segment (start 112.3 80.3) (end 112.9 80.3) (width 0.2) (layer "F.Cu") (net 1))
 (segment (start 118.75 80.25) (end 119.349 80.849) (width 0.2) (layer "F.Cu") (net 1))
 (segment (start 107.85 97.9) (end 107.999 97.751) (width 0.2) (layer "F.Cu") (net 1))
 (segment (start 115.45 96.75) (end 117.75 96.75) (width 0.2) (layer "F.Cu") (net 1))
 (segment (start 101.75 117.75) (end 102.475 117.75) (width 0.2) (layer "F.Cu") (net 1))
 (segment (start 111.5 80) (end 112 80) (width 0.2) (layer "F.Cu") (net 1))
 (segment (start 107 95.25) (end 107 94.25) (width 0.2) (layer "F.Cu") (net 1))
 (segment (start 122.549 95.951) (end 123.024452 95.951) (width 0.2) (layer "F.Cu") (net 1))
 (segment (start 119.95 84.9) (end 119.95 85.45) (width 0.2) (layer "F.Cu") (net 1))
 (segment (start 122.2 96.3) (end 122.549 95.951) (width 0.2) (layer "F.Cu") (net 1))
 (segment (start 100.025548 97.149) (end 99.75 97.424548) (width 0.2) (layer "F.Cu") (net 1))
 (segment (start 105.75 97.9) (end 105.75 96.5) (width 0.2) (layer "F.Cu") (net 1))
 (segment (start 105.75 97.9) (end 105.75 97.75) (width 0.2) (layer "F.Cu") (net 1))
 (segment (start 117.25 77.8) (end 117.25 78.15) (width 0.2) (layer "F.Cu") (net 1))
 (segment (start 122.274452 87.699) (end 122.501 87.925548) (width 0.2) (layer "F.Cu") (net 1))
 (segment (start 99.75 115.75) (end 101.75 117.75) (width 0.2) (layer "F.Cu") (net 1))
 (segment (start 123.251 95.724452) (end 123.251 93.551) (width 0.2) (layer "F.Cu") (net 1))
 (segment (start 109.949548 88.025) (end 110.475 88.025) (width 0.2) (layer "F.Cu") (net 1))
 (segment (start 105.75 94.6) (end 105.55 94.6) (width 0.2) (layer "F.Cu") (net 27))
 (segment (start 105.55 94.6) (end 101.6 90.65) (width 0.2) (layer "F.Cu") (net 27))
 (segment (start 105.5 87.35) (end 102.55 84.4) (width 0.2) (layer "F.Cu") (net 8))
 (segment (start 106.5 87.35) (end 105.5 87.35) (width 0.2) (layer "F.Cu") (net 8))
 (segment (start 104.25 77.9) (end 103.6 77.9) (width 0.2) (layer "F.Cu") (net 7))
 (segment (start 107.45 81.1) (end 104.25 77.9) (width 0.2) (layer "F.Cu") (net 7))
 (segment (start 108.5 74.6) (end 108.5 72.95) (width 0.2) (layer "F.Cu") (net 14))
 (segment (start 108.5 72.95) (end 107.05 71.5) (width 0.2) (layer "F.Cu") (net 14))
 (segment (start 110.5 76.8) (end 111.5 77.8) (width 0.2) (layer "F.Cu") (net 16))
 (segment (start 110.5 69.65) (end 110.5 76.8) (width 0.2) (layer "F.Cu") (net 16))
 (segment (start 111.95 68.2) (end 110.5 69.65) (width 0.2) (layer "F.Cu") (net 16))
 (segment (start 111.5 77.8) (end 112.35 77.8) (width 0.2) (layer "F.Cu") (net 16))
 (segment (start 116 76.25) (end 117 75.25) (width 0.2) (layer "F.Cu") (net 15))
 (segment (start 116.75 83.2) (end 116.75 80.5) (width 0.2) (layer "F.Cu") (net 15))
 (segment (start 117 74.75) (end 117.25 74.5) (width 0.2) (layer "F.Cu") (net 15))
 (segment (start 115.949 79.449) (end 115.949 77.875548) (width 0.2) (layer "F.Cu") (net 15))
 (segment (start 115.05 84.9) (end 116.75 83.2) (width 0.2) (layer "F.Cu") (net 15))
 (segment (start 115.949 77.875548) (end 116 77.824548) (width 0.2) (layer "F.Cu") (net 15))
 (segment (start 116 79.75) (end 116 79.5) (width 0.2) (layer "F.Cu") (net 15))
 (segment (start 116.75 80.5) (end 116 79.75) (width 0.2) (layer "F.Cu") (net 15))
 (segment (start 117 75.25) (end 117 74.75) (width 0.2) (layer "F.Cu") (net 15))
 (segment (start 116 77.824548) (end 116 76.25) (width 0.2) (layer "F.Cu") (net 15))
 (segment (start 116 79.5) (end 115.949 79.449) (width 0.2) (layer "F.Cu") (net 15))
 (segment (start 119.95 81.6) (end 118.5 83.05) (width 0.2) (layer "F.Cu") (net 4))
 (segment (start 118.5 89.8) (end 116.55 91.75) (width 0.2) (layer "F.Cu") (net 4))
 (segment (start 118.5 83.05) (end 118.5 89.8) (width 0.2) (layer "F.Cu") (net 4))
 (segment (start 121.45 88.45) (end 120 89.9) (width 0.2) (layer "F.Cu") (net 2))
 (segment (start 120 89.9) (end 120 95.8) (width 0.2) (layer "F.Cu") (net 2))
 (segment (start 120 95.8) (end 117.3 98.5) (width 0.2) (layer "F.Cu") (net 2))
 (segment (start 110.3 99.5) (end 109.05 98.25) (width 0.2) (layer "F.Cu") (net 29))
 (segment (start 118 99.5) (end 110.3 99.5) (width 0.2) (layer "F.Cu") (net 29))
 (segment (start 119 98.5) (end 118 99.5) (width 0.2) (layer "F.Cu") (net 29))
 (segment (start 122.05 95.2) (end 119 98.25) (width 0.2) (layer "F.Cu") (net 29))
 (segment (start 119 98.25) (end 119 98.5) (width 0.2) (layer "F.Cu") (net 29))
 (segment (start 122.2 95.2) (end 122.05 95.2) (width 0.2) (layer "F.Cu") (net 29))
 (segment (start 113.95 94.95) (end 110 91) (width 0.2) (layer "F.Cu") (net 28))
 (segment (start 110 91) (end 108.55 91) (width 0.2) (layer "F.Cu") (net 28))
 (segment (start 112.9 87.15) (end 112.9 85.2) (width 0.2) (layer "F.Cu") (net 6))
 (segment (start 113.45 87.7) (end 112.9 87.15) (width 0.2) (layer "F.Cu") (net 6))
 (segment (start 117.725 110.08) (end 122.42 110.08) (width 0.2) (layer "F.Cu") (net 17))
 (segment (start 122.42 110.08) (end 122.75 109.75) (width 0.2) (layer "F.Cu") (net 17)))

